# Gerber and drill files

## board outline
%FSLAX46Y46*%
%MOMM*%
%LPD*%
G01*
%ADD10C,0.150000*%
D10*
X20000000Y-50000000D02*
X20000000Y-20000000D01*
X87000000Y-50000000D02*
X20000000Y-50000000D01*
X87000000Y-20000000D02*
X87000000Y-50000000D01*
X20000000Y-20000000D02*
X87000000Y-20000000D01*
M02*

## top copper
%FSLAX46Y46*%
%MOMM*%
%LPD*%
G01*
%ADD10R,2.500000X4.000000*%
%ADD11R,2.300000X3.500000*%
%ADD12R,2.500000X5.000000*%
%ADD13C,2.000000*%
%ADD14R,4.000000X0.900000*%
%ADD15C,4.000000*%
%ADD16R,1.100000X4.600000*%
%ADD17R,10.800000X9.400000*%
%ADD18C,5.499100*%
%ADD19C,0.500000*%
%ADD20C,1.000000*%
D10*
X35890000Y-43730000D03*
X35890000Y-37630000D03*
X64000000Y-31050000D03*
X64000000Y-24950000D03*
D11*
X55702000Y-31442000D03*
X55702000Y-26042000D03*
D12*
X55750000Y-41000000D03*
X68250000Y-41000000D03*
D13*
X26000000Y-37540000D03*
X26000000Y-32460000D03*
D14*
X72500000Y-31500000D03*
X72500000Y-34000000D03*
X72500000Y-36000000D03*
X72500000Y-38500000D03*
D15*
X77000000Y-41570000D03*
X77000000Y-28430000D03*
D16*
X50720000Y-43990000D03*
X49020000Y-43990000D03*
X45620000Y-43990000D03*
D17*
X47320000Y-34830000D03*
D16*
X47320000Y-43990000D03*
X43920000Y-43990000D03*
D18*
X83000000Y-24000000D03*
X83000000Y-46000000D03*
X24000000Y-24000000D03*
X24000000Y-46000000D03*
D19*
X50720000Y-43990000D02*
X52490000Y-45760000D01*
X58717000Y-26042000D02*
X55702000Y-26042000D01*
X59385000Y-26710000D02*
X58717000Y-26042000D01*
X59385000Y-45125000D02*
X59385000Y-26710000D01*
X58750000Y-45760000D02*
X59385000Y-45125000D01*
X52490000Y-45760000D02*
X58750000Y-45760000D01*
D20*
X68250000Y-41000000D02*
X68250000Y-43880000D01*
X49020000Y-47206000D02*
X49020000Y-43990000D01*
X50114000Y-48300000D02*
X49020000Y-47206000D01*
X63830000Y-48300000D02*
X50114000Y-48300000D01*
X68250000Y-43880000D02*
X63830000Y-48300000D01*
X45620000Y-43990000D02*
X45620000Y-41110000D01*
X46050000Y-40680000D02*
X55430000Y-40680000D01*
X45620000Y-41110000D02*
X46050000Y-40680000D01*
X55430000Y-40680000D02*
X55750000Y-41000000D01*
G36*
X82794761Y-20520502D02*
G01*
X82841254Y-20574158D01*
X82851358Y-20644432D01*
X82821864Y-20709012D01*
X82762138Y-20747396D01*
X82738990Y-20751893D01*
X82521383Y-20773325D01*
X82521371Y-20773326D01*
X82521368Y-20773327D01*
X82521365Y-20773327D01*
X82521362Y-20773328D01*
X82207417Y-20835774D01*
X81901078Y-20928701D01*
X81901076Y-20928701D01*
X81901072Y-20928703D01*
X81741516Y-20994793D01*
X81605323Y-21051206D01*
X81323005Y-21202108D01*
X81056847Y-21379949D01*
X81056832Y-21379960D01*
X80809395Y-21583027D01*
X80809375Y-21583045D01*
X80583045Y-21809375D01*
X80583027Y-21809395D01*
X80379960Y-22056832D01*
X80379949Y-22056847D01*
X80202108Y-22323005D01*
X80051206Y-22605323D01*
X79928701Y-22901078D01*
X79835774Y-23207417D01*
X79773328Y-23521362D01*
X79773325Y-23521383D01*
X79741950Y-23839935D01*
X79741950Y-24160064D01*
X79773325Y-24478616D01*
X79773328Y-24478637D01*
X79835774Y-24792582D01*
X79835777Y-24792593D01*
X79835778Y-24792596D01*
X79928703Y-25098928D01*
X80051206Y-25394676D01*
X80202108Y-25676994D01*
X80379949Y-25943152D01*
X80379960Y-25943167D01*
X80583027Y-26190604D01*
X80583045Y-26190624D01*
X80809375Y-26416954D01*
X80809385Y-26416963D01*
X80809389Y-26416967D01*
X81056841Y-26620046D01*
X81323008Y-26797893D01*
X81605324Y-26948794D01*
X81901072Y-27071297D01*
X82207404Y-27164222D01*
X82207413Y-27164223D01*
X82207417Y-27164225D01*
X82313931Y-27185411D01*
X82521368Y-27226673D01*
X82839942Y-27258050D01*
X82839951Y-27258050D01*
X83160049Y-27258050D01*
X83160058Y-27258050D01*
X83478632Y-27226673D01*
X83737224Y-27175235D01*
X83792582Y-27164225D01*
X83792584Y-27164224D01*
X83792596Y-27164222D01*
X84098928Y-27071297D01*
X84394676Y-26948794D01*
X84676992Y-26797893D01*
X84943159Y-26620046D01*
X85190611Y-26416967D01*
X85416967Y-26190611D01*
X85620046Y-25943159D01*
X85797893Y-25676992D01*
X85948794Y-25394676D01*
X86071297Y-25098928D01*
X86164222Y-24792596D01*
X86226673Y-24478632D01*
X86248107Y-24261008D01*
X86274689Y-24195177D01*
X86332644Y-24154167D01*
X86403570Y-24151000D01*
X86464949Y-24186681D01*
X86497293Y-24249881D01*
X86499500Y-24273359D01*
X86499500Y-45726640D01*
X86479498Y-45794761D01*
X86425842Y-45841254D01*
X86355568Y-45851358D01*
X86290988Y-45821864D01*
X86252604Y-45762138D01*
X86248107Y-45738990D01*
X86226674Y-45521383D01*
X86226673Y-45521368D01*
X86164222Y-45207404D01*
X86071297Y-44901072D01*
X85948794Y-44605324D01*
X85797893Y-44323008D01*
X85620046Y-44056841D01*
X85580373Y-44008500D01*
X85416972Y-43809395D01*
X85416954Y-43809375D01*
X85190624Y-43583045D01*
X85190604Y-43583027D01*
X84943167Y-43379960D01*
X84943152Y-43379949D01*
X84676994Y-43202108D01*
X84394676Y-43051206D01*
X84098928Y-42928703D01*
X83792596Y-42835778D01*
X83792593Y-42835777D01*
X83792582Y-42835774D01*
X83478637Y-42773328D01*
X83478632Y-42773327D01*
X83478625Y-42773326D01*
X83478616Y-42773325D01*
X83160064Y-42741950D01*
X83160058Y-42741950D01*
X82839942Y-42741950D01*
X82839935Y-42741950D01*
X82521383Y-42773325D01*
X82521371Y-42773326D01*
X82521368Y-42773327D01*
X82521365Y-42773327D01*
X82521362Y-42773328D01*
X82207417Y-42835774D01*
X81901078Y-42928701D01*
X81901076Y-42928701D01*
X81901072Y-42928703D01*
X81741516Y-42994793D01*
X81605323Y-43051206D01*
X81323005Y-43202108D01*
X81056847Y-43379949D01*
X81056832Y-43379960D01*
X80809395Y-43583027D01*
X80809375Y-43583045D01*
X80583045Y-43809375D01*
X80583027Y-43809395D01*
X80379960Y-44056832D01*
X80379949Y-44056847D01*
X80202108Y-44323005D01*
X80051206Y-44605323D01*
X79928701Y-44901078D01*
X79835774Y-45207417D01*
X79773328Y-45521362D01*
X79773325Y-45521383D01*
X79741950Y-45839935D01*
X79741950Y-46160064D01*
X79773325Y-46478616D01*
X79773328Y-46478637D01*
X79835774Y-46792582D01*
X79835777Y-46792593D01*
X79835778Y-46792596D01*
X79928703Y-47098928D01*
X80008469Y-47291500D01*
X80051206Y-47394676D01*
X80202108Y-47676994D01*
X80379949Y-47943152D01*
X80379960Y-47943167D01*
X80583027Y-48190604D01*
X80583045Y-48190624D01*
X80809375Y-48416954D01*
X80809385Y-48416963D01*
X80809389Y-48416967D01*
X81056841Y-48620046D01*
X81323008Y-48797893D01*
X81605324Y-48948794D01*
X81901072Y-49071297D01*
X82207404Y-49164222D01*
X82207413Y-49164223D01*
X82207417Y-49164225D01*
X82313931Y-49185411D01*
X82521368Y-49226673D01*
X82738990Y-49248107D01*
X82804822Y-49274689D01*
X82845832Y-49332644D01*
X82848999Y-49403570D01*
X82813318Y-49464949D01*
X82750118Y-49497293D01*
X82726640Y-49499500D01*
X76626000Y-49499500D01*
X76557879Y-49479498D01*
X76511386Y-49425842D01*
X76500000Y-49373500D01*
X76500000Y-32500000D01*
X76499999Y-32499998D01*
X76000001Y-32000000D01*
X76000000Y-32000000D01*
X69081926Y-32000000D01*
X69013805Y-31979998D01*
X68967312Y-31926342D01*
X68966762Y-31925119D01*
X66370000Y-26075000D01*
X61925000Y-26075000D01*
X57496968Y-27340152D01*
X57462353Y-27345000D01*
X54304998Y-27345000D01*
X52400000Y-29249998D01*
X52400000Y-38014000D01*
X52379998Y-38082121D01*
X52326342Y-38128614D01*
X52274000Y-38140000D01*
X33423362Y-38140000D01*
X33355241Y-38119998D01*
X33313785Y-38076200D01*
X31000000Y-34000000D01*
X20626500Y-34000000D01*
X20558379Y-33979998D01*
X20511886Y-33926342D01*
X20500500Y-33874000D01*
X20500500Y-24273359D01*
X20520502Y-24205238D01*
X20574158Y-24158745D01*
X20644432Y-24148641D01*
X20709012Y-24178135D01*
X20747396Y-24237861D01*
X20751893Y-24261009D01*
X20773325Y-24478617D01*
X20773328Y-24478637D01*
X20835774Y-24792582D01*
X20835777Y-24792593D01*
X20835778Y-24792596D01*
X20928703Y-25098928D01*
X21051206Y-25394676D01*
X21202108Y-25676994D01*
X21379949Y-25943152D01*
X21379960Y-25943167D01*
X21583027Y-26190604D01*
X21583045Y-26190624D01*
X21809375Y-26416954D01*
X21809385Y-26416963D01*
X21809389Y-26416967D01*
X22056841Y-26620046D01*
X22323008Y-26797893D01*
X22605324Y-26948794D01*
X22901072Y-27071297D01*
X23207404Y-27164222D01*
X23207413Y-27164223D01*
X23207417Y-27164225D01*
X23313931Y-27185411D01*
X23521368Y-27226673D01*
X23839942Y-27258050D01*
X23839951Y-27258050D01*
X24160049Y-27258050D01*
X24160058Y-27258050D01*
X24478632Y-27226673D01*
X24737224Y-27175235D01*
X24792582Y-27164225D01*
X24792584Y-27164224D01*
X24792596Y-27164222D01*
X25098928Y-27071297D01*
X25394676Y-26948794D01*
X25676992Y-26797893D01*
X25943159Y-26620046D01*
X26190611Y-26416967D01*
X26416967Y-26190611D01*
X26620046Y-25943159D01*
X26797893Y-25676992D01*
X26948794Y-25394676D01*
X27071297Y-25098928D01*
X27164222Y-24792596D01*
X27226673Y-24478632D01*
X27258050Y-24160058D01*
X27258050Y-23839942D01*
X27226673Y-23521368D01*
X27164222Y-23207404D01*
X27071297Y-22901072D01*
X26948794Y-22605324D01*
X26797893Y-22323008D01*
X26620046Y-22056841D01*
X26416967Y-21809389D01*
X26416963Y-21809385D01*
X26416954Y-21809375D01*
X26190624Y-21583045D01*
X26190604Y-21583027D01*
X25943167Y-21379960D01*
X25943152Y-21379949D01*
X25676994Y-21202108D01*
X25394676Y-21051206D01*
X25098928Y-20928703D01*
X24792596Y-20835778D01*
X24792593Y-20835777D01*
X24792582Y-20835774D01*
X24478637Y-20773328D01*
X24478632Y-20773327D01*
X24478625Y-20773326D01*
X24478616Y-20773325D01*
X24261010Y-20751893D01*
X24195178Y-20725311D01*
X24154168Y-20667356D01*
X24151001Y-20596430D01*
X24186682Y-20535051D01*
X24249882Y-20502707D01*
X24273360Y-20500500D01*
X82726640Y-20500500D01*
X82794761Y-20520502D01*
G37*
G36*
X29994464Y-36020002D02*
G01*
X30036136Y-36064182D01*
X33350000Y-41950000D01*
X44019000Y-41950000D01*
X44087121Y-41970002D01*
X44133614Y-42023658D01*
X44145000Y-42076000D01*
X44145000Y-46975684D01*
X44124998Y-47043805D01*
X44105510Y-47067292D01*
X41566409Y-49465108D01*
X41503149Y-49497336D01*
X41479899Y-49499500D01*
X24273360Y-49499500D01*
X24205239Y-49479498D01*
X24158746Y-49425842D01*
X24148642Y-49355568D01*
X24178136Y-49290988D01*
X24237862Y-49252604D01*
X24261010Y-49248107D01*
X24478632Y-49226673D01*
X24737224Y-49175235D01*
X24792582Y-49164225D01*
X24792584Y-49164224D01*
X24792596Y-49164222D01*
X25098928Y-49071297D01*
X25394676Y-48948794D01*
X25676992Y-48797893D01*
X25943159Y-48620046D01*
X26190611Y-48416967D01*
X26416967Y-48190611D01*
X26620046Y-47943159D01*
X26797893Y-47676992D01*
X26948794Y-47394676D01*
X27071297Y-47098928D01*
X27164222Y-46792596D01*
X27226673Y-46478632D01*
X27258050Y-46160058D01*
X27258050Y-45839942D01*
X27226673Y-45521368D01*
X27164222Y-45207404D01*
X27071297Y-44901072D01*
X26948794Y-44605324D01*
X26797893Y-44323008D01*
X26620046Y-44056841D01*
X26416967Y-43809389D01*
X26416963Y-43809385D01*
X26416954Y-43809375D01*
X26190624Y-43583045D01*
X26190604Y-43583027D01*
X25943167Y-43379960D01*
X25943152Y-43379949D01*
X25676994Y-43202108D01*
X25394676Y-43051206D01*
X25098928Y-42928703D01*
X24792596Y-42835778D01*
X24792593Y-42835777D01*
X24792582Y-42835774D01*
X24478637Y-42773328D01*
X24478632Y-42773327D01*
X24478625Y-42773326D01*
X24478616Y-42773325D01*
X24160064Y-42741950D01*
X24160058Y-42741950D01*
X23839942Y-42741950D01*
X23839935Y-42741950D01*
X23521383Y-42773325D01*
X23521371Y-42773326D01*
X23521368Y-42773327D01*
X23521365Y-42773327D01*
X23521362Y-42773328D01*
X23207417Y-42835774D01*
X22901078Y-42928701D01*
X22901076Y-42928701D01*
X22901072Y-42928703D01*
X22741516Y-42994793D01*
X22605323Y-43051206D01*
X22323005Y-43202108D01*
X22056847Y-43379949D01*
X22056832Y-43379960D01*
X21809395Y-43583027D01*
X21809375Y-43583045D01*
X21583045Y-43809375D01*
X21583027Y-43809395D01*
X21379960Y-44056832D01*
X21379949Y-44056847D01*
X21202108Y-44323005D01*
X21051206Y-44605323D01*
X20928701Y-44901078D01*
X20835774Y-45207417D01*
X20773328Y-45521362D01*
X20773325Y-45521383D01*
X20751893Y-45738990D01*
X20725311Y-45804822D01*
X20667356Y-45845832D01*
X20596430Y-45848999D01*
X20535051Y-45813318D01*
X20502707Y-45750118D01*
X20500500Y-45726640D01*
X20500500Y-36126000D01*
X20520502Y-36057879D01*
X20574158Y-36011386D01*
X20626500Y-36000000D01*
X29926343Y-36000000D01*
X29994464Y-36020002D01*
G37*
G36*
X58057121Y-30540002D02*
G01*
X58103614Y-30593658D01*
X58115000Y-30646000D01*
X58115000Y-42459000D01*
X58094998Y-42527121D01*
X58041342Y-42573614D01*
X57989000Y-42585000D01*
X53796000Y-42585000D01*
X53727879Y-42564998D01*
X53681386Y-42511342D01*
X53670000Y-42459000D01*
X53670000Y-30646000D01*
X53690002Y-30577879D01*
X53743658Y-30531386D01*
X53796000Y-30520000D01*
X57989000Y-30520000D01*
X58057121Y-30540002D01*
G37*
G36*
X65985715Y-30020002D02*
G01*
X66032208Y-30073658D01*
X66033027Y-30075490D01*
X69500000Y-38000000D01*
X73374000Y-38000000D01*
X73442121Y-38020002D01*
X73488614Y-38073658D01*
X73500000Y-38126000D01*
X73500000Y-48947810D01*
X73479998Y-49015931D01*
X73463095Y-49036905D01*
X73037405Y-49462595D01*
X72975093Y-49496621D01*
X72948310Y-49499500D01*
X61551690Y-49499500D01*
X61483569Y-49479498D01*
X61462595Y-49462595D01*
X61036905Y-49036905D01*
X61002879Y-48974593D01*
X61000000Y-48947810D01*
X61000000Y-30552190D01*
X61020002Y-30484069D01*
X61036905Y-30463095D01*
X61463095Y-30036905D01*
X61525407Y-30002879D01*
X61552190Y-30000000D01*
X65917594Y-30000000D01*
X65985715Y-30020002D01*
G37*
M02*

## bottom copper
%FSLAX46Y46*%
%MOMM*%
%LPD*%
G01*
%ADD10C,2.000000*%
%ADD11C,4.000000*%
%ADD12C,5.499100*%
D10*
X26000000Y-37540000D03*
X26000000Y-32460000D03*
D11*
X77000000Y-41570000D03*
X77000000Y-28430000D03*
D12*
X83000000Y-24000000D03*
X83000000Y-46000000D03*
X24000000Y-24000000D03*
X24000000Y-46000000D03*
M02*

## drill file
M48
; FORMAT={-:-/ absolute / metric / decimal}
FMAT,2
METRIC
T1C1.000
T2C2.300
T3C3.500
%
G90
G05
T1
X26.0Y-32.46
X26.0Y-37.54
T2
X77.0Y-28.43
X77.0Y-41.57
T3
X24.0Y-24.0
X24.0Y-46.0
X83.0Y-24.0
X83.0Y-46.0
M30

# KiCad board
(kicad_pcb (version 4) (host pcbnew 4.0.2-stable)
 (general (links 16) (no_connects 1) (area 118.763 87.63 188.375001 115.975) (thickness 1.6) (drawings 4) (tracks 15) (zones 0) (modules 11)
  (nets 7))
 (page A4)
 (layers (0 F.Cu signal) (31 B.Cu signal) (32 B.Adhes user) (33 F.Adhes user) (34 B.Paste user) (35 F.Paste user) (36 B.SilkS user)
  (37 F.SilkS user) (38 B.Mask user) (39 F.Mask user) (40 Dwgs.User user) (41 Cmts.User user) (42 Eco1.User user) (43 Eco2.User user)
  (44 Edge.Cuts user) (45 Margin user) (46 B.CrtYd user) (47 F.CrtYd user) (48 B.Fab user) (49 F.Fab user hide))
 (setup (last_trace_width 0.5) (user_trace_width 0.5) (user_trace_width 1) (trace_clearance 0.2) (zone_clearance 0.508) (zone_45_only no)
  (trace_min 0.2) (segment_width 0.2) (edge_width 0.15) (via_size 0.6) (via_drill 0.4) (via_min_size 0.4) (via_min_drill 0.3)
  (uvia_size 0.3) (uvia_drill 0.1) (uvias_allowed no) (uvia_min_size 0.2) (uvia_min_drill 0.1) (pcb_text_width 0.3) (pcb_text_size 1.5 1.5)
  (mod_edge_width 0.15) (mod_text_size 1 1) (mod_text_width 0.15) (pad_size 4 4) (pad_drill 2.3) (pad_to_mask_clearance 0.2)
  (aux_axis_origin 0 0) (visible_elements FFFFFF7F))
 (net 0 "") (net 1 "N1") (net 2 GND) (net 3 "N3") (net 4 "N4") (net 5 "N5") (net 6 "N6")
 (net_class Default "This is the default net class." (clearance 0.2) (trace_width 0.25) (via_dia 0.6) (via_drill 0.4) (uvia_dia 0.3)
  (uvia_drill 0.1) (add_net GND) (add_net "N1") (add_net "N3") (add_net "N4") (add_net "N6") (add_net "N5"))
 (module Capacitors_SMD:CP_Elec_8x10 (layer F.Cu) (at 35.89 40.68 90)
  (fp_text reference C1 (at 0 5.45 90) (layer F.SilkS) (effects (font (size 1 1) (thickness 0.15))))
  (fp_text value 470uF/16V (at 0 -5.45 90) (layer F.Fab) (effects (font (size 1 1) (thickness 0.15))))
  (pad 1 smd rect (at -3.05 0 270) (size 4 2.5) (layers F.Cu F.Paste F.Mask) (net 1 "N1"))
  (pad 2 smd rect (at 3.05 0 270) (size 4 2.5) (layers F.Cu F.Paste F.Mask) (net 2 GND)))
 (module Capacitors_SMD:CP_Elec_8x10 (layer F.Cu) (at 64 28 90)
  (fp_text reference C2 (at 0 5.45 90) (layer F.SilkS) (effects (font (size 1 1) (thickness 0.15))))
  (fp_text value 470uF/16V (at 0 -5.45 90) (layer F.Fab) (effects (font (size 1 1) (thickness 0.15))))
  (pad 1 smd rect (at -3.05 0 270) (size 4 2.5) (layers F.Cu F.Paste F.Mask) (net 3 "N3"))
  (pad 2 smd rect (at 3.05 0 270) (size 4 2.5) (layers F.Cu F.Paste F.Mask) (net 2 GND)))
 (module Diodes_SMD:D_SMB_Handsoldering (layer F.Cu) (at 55.702 28.742 90)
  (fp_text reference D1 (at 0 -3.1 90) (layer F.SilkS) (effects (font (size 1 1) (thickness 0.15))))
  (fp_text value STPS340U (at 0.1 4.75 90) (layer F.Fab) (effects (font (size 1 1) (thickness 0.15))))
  (pad 1 smd rect (at -2.7 0 90) (size 3.5 2.3) (layers F.Cu F.Paste F.Mask) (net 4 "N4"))
  (pad 2 smd rect (at 2.7 0 90) (size 3.5 2.3) (layers F.Cu F.Paste F.Mask) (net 2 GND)))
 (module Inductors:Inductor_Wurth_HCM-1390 (layer F.Cu) (at 62 41)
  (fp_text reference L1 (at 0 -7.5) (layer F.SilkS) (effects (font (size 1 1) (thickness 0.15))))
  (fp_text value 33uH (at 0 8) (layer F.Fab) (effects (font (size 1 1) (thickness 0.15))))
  (pad 1 smd rect (at -6.25 0) (size 2.5 5) (layers F.Cu F.Paste F.Mask) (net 4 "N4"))
  (pad 2 smd rect (at 6.25 0) (size 2.5 5) (layers F.Cu F.Paste F.Mask) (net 3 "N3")))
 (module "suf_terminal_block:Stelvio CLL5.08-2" (layer F.Cu) (at 26 35 90)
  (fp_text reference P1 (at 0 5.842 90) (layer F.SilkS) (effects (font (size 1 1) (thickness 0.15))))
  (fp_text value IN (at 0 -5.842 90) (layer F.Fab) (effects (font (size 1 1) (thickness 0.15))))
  (pad 1 thru_hole circle (at -2.54 0 90) (size 2 2) (drill 1) (layers *.Cu *.Mask F.SilkS) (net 1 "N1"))
  (pad 2 thru_hole circle (at 2.54 0 90) (size 2 2) (drill 1) (layers *.Cu *.Mask F.SilkS) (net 2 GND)))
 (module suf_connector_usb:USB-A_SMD (layer F.Cu) (at 77 35 180)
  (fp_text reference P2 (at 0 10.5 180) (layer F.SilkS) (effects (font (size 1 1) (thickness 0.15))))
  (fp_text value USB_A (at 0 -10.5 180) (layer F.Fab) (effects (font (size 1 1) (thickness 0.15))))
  (pad 4 smd rect (at 4.5 3.5 180) (size 4 0.9) (layers F.Cu F.Paste F.Mask) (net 2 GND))
  (pad 3 smd rect (at 4.5 1 180) (size 4 0.9) (layers F.Cu F.Paste F.Mask) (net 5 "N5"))
  (pad 2 smd rect (at 4.5 -1 180) (size 4 0.9) (layers F.Cu F.Paste F.Mask) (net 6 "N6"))
  (pad 1 smd rect (at 4.5 -3.5 180) (size 4 0.9) (layers F.Cu F.Paste F.Mask) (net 3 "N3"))
  (pad 4 thru_hole circle (at 0 -6.57 180) (size 4 4) (drill 2.3) (layers *.Cu *.Mask F.SilkS) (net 2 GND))
  (pad 4 thru_hole circle (at 0 6.57 180) (size 4 4) (drill 2.3) (layers *.Cu *.Mask F.SilkS) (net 2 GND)))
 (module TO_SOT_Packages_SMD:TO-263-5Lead (layer F.Cu) (at 47.32 39.41 90)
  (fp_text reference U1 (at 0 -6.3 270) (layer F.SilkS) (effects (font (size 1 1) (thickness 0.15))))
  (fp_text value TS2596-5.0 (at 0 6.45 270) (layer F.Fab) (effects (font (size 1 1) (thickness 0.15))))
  (pad 5 smd rect (at -4.58 3.4 90) (size 4.6 1.1) (layers F.Cu F.Paste F.Mask) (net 2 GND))
  (pad 4 smd rect (at -4.58 1.7 90) (size 4.6 1.1) (layers F.Cu F.Paste F.Mask) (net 3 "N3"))
  (pad 2 smd rect (at -4.58 -1.7 90) (size 4.6 1.1) (layers F.Cu F.Paste F.Mask) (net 4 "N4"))
  (pad 3 smd rect (at 4.58 0 90) (size 9.4 10.8) (layers F.Cu F.Paste F.Mask) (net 2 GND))
  (pad 3 smd rect (at -4.58 0 90) (size 4.6 1.1) (layers F.Cu F.Paste F.Mask) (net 2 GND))
  (pad 1 smd rect (at -4.58 -3.4 90) (size 4.6 1.1) (layers F.Cu F.Paste F.Mask) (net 1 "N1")))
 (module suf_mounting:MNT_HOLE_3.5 (layer F.Cu) (at 83 24)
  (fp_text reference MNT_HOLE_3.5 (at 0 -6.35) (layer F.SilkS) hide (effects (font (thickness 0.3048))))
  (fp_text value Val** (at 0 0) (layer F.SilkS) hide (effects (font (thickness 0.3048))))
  (pad "" thru_hole circle (at 0 0) (size 5.4991 5.4991) (drill 3.50012) (layers *.Cu *.Mask F.SilkS)))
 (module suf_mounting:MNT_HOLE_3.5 (layer F.Cu) (at 83 46)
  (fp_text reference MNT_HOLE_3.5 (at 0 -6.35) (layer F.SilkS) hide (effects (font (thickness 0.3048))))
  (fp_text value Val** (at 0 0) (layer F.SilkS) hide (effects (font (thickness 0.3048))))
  (pad "" thru_hole circle (at 0 0) (size 5.4991 5.4991) (drill 3.50012) (layers *.Cu *.Mask F.SilkS)))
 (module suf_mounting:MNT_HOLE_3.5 (layer F.Cu) (at 24 24)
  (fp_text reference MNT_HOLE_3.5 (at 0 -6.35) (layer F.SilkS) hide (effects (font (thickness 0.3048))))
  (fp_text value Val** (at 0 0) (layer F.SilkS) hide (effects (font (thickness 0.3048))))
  (pad "" thru_hole circle (at 0 0) (size 5.4991 5.4991) (drill 3.50012) (layers *.Cu *.Mask F.SilkS)))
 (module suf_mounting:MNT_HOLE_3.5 (layer F.Cu) (at 24 46)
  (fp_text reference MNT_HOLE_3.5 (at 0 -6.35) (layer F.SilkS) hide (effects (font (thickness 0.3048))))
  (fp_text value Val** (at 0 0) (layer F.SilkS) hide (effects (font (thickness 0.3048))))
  (pad "" thru_hole circle (at 0 0) (size 5.4991 5.4991) (drill 3.50012) (layers *.Cu *.Mask F.SilkS)))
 (gr_line (start 20 50) (end 20 20) (angle 90) (layer Edge.Cuts) (width 0.15))
 (gr_line (start 87 50) (end 20 50) (angle 90) (layer Edge.Cuts) (width 0.15))
 (gr_line (start 87 20) (end 87 50) (angle 90) (layer Edge.Cuts) (width 0.15))
 (gr_line (start 20 20) (end 87 20) (angle 90) (layer Edge.Cuts) (width 0.15))
 (segment (start 50.72 43.99) (end 52.49 45.76) (width 0.5) (layer F.Cu) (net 2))
 (segment (start 58.717 26.042) (end 55.702 26.042) (width 0.5) (layer F.Cu) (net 2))
 (segment (start 59.385 26.71) (end 58.717 26.042) (width 0.5) (layer F.Cu) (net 2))
 (segment (start 59.385 45.125) (end 59.385 26.71) (width 0.5) (layer F.Cu) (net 2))
 (segment (start 58.75 45.76) (end 59.385 45.125) (width 0.5) (layer F.Cu) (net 2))
 (segment (start 52.49 45.76) (end 58.75 45.76) (width 0.5) (layer F.Cu) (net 2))
 (segment (start 68.25 41) (end 68.25 43.88) (width 1) (layer F.Cu) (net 3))
 (segment (start 49.02 47.206) (end 49.02 43.99) (width 1) (layer F.Cu) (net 3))
 (segment (start 50.114 48.3) (end 49.02 47.206) (width 1) (layer F.Cu) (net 3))
 (segment (start 63.83 48.3) (end 50.114 48.3) (width 1) (layer F.Cu) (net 3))
 (segment (start 68.25 43.88) (end 63.83 48.3) (width 1) (layer F.Cu) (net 3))
 (segment (start 45.62 43.99) (end 45.62 41.11) (width 1) (layer F.Cu) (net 4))
 (segment (start 46.05 40.68) (end 55.43 40.68) (width 1) (layer F.Cu) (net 4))
 (segment (start 45.62 41.11) (end 46.05 40.68) (width 1) (layer F.Cu) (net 4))
 (segment (start 55.43 40.68) (end 55.75 41) (width 1) (layer F.Cu) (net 4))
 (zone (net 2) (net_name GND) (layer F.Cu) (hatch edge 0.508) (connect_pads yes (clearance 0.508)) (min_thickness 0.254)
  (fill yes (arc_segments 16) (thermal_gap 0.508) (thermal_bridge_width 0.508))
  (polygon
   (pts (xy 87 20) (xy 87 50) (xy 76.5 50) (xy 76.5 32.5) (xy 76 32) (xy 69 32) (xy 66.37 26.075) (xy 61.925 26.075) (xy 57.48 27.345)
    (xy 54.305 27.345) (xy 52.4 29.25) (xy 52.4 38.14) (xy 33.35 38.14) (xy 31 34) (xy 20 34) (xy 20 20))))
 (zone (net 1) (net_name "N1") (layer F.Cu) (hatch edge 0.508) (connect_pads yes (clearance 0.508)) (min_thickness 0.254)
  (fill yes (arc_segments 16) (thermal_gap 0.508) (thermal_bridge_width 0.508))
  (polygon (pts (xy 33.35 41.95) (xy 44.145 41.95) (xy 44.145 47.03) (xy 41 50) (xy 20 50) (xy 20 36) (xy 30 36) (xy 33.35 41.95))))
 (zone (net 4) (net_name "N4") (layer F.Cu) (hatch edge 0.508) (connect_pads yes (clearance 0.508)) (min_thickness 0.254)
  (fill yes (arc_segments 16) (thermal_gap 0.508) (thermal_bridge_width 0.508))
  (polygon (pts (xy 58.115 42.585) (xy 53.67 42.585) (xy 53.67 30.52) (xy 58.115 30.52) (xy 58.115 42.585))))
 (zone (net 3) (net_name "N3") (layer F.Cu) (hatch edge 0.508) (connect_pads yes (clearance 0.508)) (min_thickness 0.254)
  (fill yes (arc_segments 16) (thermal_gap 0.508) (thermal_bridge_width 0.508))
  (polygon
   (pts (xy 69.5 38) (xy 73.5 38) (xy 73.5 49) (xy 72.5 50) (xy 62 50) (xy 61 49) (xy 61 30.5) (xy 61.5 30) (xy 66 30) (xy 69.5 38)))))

